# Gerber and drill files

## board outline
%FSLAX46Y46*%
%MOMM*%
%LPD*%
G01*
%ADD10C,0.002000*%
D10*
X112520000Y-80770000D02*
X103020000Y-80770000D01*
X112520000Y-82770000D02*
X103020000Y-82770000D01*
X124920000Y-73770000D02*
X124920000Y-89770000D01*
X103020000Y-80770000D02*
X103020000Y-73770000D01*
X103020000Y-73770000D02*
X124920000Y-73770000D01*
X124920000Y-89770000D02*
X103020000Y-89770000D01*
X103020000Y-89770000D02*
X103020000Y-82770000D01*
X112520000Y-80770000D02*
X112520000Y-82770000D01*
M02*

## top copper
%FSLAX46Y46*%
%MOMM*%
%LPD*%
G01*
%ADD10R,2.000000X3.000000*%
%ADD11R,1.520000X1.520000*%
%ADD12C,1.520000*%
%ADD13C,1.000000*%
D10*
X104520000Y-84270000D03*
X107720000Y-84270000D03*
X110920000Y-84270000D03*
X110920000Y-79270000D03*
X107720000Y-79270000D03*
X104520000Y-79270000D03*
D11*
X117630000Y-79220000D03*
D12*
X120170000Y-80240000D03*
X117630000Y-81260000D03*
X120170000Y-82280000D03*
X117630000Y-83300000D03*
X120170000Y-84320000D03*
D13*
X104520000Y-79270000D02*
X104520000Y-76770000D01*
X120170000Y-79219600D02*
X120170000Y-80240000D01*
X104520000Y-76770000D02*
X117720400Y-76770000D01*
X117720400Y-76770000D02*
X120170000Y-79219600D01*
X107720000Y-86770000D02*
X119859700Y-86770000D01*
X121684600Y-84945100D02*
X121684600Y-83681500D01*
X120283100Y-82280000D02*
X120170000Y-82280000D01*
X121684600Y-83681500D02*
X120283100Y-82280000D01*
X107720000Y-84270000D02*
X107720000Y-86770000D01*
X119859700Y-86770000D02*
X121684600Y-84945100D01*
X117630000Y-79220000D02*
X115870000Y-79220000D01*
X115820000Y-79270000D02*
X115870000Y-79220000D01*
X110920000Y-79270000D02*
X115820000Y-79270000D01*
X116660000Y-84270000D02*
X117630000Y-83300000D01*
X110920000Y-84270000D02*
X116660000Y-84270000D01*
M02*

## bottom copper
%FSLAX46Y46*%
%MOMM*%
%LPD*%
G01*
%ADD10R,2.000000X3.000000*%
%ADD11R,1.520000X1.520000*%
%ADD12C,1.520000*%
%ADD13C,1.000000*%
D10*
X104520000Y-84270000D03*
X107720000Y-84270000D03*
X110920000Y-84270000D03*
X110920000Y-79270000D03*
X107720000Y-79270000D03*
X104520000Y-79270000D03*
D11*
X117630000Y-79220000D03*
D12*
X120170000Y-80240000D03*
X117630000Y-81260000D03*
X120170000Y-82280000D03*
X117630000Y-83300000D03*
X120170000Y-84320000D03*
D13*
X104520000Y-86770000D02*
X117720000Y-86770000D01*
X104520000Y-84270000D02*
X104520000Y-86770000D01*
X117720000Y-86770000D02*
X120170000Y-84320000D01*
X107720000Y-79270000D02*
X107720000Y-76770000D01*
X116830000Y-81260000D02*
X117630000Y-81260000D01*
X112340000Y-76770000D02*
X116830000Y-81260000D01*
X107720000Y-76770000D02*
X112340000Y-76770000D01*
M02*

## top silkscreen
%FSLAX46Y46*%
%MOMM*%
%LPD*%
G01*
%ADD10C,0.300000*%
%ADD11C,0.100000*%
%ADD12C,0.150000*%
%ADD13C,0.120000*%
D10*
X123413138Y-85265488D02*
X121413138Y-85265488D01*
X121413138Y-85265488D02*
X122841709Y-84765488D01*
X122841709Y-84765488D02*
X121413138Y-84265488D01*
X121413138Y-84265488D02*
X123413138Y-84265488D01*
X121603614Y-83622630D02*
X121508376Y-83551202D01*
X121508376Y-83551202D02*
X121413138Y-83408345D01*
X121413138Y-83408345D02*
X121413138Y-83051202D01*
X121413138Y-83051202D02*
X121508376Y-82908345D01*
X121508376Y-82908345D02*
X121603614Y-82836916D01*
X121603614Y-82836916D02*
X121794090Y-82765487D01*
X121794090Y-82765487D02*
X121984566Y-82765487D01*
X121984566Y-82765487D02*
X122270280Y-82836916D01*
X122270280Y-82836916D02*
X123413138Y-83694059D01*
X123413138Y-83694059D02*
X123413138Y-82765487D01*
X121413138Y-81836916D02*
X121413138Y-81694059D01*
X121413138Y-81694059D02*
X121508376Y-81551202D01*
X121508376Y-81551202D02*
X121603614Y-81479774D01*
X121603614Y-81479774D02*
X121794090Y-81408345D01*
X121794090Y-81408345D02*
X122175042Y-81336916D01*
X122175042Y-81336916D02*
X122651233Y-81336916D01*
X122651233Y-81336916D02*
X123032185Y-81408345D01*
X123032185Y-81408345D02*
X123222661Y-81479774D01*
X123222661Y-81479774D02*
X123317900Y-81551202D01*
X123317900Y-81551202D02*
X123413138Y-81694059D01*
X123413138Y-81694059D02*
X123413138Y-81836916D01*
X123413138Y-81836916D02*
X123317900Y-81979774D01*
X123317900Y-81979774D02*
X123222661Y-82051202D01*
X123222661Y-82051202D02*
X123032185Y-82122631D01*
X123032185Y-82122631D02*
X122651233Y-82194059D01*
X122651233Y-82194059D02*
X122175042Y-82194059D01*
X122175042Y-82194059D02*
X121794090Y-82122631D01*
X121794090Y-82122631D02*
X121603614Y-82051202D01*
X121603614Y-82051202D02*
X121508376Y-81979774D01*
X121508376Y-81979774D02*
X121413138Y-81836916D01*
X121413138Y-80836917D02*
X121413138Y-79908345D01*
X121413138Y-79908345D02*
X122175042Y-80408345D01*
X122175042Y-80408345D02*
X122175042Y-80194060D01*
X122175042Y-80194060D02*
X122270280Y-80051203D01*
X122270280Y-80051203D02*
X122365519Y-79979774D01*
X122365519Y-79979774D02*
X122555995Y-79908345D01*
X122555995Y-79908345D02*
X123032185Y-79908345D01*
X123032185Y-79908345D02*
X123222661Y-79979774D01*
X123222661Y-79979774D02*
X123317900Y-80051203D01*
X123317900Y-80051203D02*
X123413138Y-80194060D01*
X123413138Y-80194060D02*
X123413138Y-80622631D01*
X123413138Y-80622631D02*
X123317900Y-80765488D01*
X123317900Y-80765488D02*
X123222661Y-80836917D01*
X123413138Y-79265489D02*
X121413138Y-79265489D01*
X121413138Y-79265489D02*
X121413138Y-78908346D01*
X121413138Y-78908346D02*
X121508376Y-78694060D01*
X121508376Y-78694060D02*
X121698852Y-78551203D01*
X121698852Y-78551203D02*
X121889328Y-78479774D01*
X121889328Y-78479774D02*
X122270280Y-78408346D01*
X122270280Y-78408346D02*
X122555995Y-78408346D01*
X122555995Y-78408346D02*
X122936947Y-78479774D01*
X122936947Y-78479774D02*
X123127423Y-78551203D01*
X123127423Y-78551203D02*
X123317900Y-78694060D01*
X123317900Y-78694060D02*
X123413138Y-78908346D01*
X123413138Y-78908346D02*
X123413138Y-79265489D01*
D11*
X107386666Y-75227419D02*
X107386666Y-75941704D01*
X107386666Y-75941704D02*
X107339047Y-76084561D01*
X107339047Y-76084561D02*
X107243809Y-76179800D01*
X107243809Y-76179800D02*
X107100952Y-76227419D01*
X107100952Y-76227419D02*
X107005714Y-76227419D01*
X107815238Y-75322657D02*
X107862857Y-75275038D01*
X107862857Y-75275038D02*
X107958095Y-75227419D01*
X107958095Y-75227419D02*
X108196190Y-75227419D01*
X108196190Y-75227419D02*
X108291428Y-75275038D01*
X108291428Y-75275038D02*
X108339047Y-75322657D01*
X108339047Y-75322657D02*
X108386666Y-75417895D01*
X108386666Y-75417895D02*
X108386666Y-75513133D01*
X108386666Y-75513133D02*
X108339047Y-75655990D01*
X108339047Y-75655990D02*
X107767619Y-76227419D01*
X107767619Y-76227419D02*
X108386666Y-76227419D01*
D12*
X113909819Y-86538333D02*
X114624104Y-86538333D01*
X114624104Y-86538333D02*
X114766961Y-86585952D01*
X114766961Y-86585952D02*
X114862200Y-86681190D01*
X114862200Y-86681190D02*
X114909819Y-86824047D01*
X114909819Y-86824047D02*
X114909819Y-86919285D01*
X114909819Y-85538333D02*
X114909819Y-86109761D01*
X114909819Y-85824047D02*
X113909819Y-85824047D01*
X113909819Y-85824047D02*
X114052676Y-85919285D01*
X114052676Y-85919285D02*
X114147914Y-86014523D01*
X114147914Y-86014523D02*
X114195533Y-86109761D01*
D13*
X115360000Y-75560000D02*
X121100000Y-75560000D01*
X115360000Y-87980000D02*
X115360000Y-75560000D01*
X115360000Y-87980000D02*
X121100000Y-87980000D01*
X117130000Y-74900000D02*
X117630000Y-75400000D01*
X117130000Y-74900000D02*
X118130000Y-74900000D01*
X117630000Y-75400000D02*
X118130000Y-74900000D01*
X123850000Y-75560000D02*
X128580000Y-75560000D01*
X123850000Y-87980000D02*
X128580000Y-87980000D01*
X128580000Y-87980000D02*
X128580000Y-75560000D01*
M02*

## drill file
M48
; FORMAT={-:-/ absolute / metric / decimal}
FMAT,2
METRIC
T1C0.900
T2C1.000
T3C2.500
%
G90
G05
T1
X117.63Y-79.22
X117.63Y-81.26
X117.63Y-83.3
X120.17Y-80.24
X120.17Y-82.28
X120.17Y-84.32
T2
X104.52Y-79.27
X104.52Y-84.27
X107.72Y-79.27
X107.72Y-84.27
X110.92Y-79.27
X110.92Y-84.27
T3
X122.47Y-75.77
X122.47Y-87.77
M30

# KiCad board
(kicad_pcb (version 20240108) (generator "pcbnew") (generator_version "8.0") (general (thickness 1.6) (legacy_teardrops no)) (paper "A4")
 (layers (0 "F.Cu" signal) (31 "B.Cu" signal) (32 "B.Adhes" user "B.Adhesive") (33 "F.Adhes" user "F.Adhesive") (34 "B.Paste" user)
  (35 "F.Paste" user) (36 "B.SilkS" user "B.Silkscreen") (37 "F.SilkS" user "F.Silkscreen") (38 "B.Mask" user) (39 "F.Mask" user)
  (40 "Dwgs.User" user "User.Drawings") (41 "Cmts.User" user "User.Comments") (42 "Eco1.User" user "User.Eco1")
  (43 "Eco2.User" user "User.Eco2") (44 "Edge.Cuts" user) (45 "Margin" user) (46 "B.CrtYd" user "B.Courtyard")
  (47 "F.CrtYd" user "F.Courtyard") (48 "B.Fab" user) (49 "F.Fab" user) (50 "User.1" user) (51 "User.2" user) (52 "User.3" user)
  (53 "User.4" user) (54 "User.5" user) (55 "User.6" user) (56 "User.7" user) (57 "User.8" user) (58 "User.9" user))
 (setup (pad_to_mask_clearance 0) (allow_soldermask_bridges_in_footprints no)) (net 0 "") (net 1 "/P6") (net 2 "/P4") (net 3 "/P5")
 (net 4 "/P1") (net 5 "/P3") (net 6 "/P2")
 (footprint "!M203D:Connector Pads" (layer "F.Cu") (at 107.72 81.77)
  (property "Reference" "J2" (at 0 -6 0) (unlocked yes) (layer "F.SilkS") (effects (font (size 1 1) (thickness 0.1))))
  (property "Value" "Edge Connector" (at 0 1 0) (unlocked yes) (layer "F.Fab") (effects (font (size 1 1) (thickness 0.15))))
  (pad "1" thru_hole rect (at -3.2 2.5) (size 2 3) (drill 1) (layers "*.Cu" "*.Mask") (remove_unused_layers no) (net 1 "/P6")
   (thermal_bridge_angle 45))
  (pad "2" thru_hole rect (at 0 2.5) (size 2 3) (drill 1) (layers "*.Cu" "*.Mask") (remove_unused_layers no) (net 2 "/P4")
   (thermal_bridge_angle 45))
  (pad "3" thru_hole rect (at 3.2 2.5) (size 2 3) (drill 1) (layers "*.Cu" "*.Mask") (remove_unused_layers no) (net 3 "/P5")
   (thermal_bridge_angle 45))
  (pad "4" thru_hole rect (at 3.2 -2.5) (size 2 3) (drill 1) (layers "*.Cu" "*.Mask") (remove_unused_layers no) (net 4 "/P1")
   (thermal_bridge_angle 45))
  (pad "5" thru_hole rect (at 0 -2.5) (size 2 3) (drill 1) (layers "*.Cu" "*.Mask") (remove_unused_layers no) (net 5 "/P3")
   (thermal_bridge_angle 45))
  (pad "6" thru_hole rect (at -3.2 -2.5) (size 2 3) (drill 1) (layers "*.Cu" "*.Mask") (remove_unused_layers no) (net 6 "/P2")
   (thermal_bridge_angle 45)))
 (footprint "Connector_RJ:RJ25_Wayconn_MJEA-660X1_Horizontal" (layer "F.Cu") (at 117.63 79.22 90)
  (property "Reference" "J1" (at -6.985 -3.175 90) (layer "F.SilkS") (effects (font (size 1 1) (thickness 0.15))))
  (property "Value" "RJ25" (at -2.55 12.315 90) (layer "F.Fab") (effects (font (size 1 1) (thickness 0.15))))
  (fp_line (start 3.66 -2.27) (end 3.66 3.47) (stroke (width 0.12) (type solid)) (layer "F.SilkS"))
  (fp_line (start -8.76 -2.27) (end 3.66 -2.27) (stroke (width 0.12) (type solid)) (layer "F.SilkS"))
  (fp_line (start -8.76 -2.27) (end -8.76 3.47) (stroke (width 0.12) (type solid)) (layer "F.SilkS"))
  (fp_line (start 4.32 -0.5) (end 3.82 0) (stroke (width 0.12) (type solid)) (layer "F.SilkS"))
  (fp_line (start 4.32 -0.5) (end 4.32 0.5) (stroke (width 0.12) (type solid)) (layer "F.SilkS"))
  (fp_line (start 3.82 0) (end 4.32 0.5) (stroke (width 0.12) (type solid)) (layer "F.SilkS"))
  (fp_line (start 3.66 6.22) (end 3.66 10.95) (stroke (width 0.12) (type solid)) (layer "F.SilkS"))
  (fp_line (start -8.76 6.22) (end -8.76 10.95) (stroke (width 0.12) (type solid)) (layer "F.SilkS"))
  (fp_line (start -8.76 10.95) (end 3.66 10.95) (stroke (width 0.12) (type solid)) (layer "F.SilkS"))
  (pad "" np_thru_hole circle (at -8.55 4.84 90) (size 2.5 2.5) (drill 2.5) (layers "F&B.Cu" "*.Mask"))
  (pad "" np_thru_hole circle (at 3.45 4.84 90) (size 2.5 2.5) (drill 2.5) (layers "F&B.Cu" "*.Mask"))
  (pad "1" thru_hole rect (at 0 0 90) (size 1.52 1.52) (drill 0.9) (layers "*.Cu" "*.Mask") (remove_unused_layers no) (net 4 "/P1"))
  (pad "2" thru_hole circle (at -1.02 2.54 90) (size 1.52 1.52) (drill 0.9) (layers "*.Cu" "*.Mask") (remove_unused_layers no) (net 6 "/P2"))
  (pad "3" thru_hole circle (at -2.04 0 90) (size 1.52 1.52) (drill 0.9) (layers "*.Cu" "*.Mask") (remove_unused_layers no) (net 5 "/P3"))
  (pad "4" thru_hole circle (at -3.06 2.54 90) (size 1.52 1.52) (drill 0.9) (layers "*.Cu" "*.Mask") (remove_unused_layers no) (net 2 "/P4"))
  (pad "5" thru_hole circle (at -4.08 0 90) (size 1.52 1.52) (drill 0.9) (layers "*.Cu" "*.Mask") (remove_unused_layers no) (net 3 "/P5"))
  (pad "6" thru_hole circle (at -5.1 2.54 90) (size 1.52 1.52) (drill 0.9) (layers "*.Cu" "*.Mask") (remove_unused_layers no) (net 1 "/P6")))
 (gr_line (start 112.52 80.77) (end 103.02 80.77) (stroke (width 0.002) (type default)) (layer "Edge.Cuts"))
 (gr_line (start 112.52 82.77) (end 103.02 82.77) (stroke (width 0.002) (type default)) (layer "Edge.Cuts"))
 (gr_line (start 124.92 73.77) (end 124.92 89.77) (stroke (width 0.002) (type default)) (layer "Edge.Cuts"))
 (gr_line (start 103.02 80.77) (end 103.02 73.77) (stroke (width 0.002) (type default)) (layer "Edge.Cuts"))
 (gr_line (start 103.02 73.77) (end 124.92 73.77) (stroke (width 0.002) (type default)) (layer "Edge.Cuts"))
 (gr_line (start 124.92 89.77) (end 103.02 89.77) (stroke (width 0.002) (type default)) (layer "Edge.Cuts"))
 (gr_line (start 103.02 89.77) (end 103.02 82.77) (stroke (width 0.002) (type default)) (layer "Edge.Cuts"))
 (gr_line (start 112.52 80.77) (end 112.52 82.77) (stroke (width 0.002) (type default)) (layer "Edge.Cuts"))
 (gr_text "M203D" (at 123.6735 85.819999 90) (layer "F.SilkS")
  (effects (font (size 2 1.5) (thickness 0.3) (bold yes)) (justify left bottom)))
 (segment (start 104.52 79.27) (end 104.52 76.77) (width 1) (layer "F.Cu") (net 6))
 (segment (start 120.17 79.2196) (end 120.17 80.24) (width 1) (layer "F.Cu") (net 6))
 (segment (start 104.52 76.77) (end 117.7204 76.77) (width 1) (layer "F.Cu") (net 6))
 (segment (start 117.7204 76.77) (end 120.17 79.2196) (width 1) (layer "F.Cu") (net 6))
 (segment (start 104.52 86.77) (end 117.72 86.77) (width 1) (layer "B.Cu") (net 1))
 (segment (start 104.52 84.27) (end 104.52 86.77) (width 1) (layer "B.Cu") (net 1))
 (segment (start 117.72 86.77) (end 120.17 84.32) (width 1) (layer "B.Cu") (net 1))
 (segment (start 107.72 79.27) (end 107.72 76.77) (width 1) (layer "B.Cu") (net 5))
 (segment (start 116.83 81.26) (end 117.63 81.26) (width 1) (layer "B.Cu") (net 5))
 (segment (start 112.34 76.77) (end 116.83 81.26) (width 1) (layer "B.Cu") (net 5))
 (segment (start 107.72 76.77) (end 112.34 76.77) (width 1) (layer "B.Cu") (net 5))
 (segment (start 107.72 86.77) (end 119.8597 86.77) (width 1) (layer "F.Cu") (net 2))
 (segment (start 121.6846 84.9451) (end 121.6846 83.6815) (width 1) (layer "F.Cu") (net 2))
 (segment (start 120.2831 82.28) (end 120.17 82.28) (width 1) (layer "F.Cu") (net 2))
 (segment (start 121.6846 83.6815) (end 120.2831 82.28) (width 1) (layer "F.Cu") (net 2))
 (segment (start 107.72 84.27) (end 107.72 86.77) (width 1) (layer "F.Cu") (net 2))
 (segment (start 119.8597 86.77) (end 121.6846 84.9451) (width 1) (layer "F.Cu") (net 2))
 (segment (start 117.63 79.22) (end 115.87 79.22) (width 1) (layer "F.Cu") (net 4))
 (segment (start 115.82 79.27) (end 115.87 79.22) (width 1) (layer "F.Cu") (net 4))
 (segment (start 110.92 79.27) (end 115.82 79.27) (width 1) (layer "F.Cu") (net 4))
 (segment (start 116.66 84.27) (end 117.63 83.3) (width 1) (layer "F.Cu") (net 3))
 (segment (start 110.92 84.27) (end 116.66 84.27) (width 1) (layer "F.Cu") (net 3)))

